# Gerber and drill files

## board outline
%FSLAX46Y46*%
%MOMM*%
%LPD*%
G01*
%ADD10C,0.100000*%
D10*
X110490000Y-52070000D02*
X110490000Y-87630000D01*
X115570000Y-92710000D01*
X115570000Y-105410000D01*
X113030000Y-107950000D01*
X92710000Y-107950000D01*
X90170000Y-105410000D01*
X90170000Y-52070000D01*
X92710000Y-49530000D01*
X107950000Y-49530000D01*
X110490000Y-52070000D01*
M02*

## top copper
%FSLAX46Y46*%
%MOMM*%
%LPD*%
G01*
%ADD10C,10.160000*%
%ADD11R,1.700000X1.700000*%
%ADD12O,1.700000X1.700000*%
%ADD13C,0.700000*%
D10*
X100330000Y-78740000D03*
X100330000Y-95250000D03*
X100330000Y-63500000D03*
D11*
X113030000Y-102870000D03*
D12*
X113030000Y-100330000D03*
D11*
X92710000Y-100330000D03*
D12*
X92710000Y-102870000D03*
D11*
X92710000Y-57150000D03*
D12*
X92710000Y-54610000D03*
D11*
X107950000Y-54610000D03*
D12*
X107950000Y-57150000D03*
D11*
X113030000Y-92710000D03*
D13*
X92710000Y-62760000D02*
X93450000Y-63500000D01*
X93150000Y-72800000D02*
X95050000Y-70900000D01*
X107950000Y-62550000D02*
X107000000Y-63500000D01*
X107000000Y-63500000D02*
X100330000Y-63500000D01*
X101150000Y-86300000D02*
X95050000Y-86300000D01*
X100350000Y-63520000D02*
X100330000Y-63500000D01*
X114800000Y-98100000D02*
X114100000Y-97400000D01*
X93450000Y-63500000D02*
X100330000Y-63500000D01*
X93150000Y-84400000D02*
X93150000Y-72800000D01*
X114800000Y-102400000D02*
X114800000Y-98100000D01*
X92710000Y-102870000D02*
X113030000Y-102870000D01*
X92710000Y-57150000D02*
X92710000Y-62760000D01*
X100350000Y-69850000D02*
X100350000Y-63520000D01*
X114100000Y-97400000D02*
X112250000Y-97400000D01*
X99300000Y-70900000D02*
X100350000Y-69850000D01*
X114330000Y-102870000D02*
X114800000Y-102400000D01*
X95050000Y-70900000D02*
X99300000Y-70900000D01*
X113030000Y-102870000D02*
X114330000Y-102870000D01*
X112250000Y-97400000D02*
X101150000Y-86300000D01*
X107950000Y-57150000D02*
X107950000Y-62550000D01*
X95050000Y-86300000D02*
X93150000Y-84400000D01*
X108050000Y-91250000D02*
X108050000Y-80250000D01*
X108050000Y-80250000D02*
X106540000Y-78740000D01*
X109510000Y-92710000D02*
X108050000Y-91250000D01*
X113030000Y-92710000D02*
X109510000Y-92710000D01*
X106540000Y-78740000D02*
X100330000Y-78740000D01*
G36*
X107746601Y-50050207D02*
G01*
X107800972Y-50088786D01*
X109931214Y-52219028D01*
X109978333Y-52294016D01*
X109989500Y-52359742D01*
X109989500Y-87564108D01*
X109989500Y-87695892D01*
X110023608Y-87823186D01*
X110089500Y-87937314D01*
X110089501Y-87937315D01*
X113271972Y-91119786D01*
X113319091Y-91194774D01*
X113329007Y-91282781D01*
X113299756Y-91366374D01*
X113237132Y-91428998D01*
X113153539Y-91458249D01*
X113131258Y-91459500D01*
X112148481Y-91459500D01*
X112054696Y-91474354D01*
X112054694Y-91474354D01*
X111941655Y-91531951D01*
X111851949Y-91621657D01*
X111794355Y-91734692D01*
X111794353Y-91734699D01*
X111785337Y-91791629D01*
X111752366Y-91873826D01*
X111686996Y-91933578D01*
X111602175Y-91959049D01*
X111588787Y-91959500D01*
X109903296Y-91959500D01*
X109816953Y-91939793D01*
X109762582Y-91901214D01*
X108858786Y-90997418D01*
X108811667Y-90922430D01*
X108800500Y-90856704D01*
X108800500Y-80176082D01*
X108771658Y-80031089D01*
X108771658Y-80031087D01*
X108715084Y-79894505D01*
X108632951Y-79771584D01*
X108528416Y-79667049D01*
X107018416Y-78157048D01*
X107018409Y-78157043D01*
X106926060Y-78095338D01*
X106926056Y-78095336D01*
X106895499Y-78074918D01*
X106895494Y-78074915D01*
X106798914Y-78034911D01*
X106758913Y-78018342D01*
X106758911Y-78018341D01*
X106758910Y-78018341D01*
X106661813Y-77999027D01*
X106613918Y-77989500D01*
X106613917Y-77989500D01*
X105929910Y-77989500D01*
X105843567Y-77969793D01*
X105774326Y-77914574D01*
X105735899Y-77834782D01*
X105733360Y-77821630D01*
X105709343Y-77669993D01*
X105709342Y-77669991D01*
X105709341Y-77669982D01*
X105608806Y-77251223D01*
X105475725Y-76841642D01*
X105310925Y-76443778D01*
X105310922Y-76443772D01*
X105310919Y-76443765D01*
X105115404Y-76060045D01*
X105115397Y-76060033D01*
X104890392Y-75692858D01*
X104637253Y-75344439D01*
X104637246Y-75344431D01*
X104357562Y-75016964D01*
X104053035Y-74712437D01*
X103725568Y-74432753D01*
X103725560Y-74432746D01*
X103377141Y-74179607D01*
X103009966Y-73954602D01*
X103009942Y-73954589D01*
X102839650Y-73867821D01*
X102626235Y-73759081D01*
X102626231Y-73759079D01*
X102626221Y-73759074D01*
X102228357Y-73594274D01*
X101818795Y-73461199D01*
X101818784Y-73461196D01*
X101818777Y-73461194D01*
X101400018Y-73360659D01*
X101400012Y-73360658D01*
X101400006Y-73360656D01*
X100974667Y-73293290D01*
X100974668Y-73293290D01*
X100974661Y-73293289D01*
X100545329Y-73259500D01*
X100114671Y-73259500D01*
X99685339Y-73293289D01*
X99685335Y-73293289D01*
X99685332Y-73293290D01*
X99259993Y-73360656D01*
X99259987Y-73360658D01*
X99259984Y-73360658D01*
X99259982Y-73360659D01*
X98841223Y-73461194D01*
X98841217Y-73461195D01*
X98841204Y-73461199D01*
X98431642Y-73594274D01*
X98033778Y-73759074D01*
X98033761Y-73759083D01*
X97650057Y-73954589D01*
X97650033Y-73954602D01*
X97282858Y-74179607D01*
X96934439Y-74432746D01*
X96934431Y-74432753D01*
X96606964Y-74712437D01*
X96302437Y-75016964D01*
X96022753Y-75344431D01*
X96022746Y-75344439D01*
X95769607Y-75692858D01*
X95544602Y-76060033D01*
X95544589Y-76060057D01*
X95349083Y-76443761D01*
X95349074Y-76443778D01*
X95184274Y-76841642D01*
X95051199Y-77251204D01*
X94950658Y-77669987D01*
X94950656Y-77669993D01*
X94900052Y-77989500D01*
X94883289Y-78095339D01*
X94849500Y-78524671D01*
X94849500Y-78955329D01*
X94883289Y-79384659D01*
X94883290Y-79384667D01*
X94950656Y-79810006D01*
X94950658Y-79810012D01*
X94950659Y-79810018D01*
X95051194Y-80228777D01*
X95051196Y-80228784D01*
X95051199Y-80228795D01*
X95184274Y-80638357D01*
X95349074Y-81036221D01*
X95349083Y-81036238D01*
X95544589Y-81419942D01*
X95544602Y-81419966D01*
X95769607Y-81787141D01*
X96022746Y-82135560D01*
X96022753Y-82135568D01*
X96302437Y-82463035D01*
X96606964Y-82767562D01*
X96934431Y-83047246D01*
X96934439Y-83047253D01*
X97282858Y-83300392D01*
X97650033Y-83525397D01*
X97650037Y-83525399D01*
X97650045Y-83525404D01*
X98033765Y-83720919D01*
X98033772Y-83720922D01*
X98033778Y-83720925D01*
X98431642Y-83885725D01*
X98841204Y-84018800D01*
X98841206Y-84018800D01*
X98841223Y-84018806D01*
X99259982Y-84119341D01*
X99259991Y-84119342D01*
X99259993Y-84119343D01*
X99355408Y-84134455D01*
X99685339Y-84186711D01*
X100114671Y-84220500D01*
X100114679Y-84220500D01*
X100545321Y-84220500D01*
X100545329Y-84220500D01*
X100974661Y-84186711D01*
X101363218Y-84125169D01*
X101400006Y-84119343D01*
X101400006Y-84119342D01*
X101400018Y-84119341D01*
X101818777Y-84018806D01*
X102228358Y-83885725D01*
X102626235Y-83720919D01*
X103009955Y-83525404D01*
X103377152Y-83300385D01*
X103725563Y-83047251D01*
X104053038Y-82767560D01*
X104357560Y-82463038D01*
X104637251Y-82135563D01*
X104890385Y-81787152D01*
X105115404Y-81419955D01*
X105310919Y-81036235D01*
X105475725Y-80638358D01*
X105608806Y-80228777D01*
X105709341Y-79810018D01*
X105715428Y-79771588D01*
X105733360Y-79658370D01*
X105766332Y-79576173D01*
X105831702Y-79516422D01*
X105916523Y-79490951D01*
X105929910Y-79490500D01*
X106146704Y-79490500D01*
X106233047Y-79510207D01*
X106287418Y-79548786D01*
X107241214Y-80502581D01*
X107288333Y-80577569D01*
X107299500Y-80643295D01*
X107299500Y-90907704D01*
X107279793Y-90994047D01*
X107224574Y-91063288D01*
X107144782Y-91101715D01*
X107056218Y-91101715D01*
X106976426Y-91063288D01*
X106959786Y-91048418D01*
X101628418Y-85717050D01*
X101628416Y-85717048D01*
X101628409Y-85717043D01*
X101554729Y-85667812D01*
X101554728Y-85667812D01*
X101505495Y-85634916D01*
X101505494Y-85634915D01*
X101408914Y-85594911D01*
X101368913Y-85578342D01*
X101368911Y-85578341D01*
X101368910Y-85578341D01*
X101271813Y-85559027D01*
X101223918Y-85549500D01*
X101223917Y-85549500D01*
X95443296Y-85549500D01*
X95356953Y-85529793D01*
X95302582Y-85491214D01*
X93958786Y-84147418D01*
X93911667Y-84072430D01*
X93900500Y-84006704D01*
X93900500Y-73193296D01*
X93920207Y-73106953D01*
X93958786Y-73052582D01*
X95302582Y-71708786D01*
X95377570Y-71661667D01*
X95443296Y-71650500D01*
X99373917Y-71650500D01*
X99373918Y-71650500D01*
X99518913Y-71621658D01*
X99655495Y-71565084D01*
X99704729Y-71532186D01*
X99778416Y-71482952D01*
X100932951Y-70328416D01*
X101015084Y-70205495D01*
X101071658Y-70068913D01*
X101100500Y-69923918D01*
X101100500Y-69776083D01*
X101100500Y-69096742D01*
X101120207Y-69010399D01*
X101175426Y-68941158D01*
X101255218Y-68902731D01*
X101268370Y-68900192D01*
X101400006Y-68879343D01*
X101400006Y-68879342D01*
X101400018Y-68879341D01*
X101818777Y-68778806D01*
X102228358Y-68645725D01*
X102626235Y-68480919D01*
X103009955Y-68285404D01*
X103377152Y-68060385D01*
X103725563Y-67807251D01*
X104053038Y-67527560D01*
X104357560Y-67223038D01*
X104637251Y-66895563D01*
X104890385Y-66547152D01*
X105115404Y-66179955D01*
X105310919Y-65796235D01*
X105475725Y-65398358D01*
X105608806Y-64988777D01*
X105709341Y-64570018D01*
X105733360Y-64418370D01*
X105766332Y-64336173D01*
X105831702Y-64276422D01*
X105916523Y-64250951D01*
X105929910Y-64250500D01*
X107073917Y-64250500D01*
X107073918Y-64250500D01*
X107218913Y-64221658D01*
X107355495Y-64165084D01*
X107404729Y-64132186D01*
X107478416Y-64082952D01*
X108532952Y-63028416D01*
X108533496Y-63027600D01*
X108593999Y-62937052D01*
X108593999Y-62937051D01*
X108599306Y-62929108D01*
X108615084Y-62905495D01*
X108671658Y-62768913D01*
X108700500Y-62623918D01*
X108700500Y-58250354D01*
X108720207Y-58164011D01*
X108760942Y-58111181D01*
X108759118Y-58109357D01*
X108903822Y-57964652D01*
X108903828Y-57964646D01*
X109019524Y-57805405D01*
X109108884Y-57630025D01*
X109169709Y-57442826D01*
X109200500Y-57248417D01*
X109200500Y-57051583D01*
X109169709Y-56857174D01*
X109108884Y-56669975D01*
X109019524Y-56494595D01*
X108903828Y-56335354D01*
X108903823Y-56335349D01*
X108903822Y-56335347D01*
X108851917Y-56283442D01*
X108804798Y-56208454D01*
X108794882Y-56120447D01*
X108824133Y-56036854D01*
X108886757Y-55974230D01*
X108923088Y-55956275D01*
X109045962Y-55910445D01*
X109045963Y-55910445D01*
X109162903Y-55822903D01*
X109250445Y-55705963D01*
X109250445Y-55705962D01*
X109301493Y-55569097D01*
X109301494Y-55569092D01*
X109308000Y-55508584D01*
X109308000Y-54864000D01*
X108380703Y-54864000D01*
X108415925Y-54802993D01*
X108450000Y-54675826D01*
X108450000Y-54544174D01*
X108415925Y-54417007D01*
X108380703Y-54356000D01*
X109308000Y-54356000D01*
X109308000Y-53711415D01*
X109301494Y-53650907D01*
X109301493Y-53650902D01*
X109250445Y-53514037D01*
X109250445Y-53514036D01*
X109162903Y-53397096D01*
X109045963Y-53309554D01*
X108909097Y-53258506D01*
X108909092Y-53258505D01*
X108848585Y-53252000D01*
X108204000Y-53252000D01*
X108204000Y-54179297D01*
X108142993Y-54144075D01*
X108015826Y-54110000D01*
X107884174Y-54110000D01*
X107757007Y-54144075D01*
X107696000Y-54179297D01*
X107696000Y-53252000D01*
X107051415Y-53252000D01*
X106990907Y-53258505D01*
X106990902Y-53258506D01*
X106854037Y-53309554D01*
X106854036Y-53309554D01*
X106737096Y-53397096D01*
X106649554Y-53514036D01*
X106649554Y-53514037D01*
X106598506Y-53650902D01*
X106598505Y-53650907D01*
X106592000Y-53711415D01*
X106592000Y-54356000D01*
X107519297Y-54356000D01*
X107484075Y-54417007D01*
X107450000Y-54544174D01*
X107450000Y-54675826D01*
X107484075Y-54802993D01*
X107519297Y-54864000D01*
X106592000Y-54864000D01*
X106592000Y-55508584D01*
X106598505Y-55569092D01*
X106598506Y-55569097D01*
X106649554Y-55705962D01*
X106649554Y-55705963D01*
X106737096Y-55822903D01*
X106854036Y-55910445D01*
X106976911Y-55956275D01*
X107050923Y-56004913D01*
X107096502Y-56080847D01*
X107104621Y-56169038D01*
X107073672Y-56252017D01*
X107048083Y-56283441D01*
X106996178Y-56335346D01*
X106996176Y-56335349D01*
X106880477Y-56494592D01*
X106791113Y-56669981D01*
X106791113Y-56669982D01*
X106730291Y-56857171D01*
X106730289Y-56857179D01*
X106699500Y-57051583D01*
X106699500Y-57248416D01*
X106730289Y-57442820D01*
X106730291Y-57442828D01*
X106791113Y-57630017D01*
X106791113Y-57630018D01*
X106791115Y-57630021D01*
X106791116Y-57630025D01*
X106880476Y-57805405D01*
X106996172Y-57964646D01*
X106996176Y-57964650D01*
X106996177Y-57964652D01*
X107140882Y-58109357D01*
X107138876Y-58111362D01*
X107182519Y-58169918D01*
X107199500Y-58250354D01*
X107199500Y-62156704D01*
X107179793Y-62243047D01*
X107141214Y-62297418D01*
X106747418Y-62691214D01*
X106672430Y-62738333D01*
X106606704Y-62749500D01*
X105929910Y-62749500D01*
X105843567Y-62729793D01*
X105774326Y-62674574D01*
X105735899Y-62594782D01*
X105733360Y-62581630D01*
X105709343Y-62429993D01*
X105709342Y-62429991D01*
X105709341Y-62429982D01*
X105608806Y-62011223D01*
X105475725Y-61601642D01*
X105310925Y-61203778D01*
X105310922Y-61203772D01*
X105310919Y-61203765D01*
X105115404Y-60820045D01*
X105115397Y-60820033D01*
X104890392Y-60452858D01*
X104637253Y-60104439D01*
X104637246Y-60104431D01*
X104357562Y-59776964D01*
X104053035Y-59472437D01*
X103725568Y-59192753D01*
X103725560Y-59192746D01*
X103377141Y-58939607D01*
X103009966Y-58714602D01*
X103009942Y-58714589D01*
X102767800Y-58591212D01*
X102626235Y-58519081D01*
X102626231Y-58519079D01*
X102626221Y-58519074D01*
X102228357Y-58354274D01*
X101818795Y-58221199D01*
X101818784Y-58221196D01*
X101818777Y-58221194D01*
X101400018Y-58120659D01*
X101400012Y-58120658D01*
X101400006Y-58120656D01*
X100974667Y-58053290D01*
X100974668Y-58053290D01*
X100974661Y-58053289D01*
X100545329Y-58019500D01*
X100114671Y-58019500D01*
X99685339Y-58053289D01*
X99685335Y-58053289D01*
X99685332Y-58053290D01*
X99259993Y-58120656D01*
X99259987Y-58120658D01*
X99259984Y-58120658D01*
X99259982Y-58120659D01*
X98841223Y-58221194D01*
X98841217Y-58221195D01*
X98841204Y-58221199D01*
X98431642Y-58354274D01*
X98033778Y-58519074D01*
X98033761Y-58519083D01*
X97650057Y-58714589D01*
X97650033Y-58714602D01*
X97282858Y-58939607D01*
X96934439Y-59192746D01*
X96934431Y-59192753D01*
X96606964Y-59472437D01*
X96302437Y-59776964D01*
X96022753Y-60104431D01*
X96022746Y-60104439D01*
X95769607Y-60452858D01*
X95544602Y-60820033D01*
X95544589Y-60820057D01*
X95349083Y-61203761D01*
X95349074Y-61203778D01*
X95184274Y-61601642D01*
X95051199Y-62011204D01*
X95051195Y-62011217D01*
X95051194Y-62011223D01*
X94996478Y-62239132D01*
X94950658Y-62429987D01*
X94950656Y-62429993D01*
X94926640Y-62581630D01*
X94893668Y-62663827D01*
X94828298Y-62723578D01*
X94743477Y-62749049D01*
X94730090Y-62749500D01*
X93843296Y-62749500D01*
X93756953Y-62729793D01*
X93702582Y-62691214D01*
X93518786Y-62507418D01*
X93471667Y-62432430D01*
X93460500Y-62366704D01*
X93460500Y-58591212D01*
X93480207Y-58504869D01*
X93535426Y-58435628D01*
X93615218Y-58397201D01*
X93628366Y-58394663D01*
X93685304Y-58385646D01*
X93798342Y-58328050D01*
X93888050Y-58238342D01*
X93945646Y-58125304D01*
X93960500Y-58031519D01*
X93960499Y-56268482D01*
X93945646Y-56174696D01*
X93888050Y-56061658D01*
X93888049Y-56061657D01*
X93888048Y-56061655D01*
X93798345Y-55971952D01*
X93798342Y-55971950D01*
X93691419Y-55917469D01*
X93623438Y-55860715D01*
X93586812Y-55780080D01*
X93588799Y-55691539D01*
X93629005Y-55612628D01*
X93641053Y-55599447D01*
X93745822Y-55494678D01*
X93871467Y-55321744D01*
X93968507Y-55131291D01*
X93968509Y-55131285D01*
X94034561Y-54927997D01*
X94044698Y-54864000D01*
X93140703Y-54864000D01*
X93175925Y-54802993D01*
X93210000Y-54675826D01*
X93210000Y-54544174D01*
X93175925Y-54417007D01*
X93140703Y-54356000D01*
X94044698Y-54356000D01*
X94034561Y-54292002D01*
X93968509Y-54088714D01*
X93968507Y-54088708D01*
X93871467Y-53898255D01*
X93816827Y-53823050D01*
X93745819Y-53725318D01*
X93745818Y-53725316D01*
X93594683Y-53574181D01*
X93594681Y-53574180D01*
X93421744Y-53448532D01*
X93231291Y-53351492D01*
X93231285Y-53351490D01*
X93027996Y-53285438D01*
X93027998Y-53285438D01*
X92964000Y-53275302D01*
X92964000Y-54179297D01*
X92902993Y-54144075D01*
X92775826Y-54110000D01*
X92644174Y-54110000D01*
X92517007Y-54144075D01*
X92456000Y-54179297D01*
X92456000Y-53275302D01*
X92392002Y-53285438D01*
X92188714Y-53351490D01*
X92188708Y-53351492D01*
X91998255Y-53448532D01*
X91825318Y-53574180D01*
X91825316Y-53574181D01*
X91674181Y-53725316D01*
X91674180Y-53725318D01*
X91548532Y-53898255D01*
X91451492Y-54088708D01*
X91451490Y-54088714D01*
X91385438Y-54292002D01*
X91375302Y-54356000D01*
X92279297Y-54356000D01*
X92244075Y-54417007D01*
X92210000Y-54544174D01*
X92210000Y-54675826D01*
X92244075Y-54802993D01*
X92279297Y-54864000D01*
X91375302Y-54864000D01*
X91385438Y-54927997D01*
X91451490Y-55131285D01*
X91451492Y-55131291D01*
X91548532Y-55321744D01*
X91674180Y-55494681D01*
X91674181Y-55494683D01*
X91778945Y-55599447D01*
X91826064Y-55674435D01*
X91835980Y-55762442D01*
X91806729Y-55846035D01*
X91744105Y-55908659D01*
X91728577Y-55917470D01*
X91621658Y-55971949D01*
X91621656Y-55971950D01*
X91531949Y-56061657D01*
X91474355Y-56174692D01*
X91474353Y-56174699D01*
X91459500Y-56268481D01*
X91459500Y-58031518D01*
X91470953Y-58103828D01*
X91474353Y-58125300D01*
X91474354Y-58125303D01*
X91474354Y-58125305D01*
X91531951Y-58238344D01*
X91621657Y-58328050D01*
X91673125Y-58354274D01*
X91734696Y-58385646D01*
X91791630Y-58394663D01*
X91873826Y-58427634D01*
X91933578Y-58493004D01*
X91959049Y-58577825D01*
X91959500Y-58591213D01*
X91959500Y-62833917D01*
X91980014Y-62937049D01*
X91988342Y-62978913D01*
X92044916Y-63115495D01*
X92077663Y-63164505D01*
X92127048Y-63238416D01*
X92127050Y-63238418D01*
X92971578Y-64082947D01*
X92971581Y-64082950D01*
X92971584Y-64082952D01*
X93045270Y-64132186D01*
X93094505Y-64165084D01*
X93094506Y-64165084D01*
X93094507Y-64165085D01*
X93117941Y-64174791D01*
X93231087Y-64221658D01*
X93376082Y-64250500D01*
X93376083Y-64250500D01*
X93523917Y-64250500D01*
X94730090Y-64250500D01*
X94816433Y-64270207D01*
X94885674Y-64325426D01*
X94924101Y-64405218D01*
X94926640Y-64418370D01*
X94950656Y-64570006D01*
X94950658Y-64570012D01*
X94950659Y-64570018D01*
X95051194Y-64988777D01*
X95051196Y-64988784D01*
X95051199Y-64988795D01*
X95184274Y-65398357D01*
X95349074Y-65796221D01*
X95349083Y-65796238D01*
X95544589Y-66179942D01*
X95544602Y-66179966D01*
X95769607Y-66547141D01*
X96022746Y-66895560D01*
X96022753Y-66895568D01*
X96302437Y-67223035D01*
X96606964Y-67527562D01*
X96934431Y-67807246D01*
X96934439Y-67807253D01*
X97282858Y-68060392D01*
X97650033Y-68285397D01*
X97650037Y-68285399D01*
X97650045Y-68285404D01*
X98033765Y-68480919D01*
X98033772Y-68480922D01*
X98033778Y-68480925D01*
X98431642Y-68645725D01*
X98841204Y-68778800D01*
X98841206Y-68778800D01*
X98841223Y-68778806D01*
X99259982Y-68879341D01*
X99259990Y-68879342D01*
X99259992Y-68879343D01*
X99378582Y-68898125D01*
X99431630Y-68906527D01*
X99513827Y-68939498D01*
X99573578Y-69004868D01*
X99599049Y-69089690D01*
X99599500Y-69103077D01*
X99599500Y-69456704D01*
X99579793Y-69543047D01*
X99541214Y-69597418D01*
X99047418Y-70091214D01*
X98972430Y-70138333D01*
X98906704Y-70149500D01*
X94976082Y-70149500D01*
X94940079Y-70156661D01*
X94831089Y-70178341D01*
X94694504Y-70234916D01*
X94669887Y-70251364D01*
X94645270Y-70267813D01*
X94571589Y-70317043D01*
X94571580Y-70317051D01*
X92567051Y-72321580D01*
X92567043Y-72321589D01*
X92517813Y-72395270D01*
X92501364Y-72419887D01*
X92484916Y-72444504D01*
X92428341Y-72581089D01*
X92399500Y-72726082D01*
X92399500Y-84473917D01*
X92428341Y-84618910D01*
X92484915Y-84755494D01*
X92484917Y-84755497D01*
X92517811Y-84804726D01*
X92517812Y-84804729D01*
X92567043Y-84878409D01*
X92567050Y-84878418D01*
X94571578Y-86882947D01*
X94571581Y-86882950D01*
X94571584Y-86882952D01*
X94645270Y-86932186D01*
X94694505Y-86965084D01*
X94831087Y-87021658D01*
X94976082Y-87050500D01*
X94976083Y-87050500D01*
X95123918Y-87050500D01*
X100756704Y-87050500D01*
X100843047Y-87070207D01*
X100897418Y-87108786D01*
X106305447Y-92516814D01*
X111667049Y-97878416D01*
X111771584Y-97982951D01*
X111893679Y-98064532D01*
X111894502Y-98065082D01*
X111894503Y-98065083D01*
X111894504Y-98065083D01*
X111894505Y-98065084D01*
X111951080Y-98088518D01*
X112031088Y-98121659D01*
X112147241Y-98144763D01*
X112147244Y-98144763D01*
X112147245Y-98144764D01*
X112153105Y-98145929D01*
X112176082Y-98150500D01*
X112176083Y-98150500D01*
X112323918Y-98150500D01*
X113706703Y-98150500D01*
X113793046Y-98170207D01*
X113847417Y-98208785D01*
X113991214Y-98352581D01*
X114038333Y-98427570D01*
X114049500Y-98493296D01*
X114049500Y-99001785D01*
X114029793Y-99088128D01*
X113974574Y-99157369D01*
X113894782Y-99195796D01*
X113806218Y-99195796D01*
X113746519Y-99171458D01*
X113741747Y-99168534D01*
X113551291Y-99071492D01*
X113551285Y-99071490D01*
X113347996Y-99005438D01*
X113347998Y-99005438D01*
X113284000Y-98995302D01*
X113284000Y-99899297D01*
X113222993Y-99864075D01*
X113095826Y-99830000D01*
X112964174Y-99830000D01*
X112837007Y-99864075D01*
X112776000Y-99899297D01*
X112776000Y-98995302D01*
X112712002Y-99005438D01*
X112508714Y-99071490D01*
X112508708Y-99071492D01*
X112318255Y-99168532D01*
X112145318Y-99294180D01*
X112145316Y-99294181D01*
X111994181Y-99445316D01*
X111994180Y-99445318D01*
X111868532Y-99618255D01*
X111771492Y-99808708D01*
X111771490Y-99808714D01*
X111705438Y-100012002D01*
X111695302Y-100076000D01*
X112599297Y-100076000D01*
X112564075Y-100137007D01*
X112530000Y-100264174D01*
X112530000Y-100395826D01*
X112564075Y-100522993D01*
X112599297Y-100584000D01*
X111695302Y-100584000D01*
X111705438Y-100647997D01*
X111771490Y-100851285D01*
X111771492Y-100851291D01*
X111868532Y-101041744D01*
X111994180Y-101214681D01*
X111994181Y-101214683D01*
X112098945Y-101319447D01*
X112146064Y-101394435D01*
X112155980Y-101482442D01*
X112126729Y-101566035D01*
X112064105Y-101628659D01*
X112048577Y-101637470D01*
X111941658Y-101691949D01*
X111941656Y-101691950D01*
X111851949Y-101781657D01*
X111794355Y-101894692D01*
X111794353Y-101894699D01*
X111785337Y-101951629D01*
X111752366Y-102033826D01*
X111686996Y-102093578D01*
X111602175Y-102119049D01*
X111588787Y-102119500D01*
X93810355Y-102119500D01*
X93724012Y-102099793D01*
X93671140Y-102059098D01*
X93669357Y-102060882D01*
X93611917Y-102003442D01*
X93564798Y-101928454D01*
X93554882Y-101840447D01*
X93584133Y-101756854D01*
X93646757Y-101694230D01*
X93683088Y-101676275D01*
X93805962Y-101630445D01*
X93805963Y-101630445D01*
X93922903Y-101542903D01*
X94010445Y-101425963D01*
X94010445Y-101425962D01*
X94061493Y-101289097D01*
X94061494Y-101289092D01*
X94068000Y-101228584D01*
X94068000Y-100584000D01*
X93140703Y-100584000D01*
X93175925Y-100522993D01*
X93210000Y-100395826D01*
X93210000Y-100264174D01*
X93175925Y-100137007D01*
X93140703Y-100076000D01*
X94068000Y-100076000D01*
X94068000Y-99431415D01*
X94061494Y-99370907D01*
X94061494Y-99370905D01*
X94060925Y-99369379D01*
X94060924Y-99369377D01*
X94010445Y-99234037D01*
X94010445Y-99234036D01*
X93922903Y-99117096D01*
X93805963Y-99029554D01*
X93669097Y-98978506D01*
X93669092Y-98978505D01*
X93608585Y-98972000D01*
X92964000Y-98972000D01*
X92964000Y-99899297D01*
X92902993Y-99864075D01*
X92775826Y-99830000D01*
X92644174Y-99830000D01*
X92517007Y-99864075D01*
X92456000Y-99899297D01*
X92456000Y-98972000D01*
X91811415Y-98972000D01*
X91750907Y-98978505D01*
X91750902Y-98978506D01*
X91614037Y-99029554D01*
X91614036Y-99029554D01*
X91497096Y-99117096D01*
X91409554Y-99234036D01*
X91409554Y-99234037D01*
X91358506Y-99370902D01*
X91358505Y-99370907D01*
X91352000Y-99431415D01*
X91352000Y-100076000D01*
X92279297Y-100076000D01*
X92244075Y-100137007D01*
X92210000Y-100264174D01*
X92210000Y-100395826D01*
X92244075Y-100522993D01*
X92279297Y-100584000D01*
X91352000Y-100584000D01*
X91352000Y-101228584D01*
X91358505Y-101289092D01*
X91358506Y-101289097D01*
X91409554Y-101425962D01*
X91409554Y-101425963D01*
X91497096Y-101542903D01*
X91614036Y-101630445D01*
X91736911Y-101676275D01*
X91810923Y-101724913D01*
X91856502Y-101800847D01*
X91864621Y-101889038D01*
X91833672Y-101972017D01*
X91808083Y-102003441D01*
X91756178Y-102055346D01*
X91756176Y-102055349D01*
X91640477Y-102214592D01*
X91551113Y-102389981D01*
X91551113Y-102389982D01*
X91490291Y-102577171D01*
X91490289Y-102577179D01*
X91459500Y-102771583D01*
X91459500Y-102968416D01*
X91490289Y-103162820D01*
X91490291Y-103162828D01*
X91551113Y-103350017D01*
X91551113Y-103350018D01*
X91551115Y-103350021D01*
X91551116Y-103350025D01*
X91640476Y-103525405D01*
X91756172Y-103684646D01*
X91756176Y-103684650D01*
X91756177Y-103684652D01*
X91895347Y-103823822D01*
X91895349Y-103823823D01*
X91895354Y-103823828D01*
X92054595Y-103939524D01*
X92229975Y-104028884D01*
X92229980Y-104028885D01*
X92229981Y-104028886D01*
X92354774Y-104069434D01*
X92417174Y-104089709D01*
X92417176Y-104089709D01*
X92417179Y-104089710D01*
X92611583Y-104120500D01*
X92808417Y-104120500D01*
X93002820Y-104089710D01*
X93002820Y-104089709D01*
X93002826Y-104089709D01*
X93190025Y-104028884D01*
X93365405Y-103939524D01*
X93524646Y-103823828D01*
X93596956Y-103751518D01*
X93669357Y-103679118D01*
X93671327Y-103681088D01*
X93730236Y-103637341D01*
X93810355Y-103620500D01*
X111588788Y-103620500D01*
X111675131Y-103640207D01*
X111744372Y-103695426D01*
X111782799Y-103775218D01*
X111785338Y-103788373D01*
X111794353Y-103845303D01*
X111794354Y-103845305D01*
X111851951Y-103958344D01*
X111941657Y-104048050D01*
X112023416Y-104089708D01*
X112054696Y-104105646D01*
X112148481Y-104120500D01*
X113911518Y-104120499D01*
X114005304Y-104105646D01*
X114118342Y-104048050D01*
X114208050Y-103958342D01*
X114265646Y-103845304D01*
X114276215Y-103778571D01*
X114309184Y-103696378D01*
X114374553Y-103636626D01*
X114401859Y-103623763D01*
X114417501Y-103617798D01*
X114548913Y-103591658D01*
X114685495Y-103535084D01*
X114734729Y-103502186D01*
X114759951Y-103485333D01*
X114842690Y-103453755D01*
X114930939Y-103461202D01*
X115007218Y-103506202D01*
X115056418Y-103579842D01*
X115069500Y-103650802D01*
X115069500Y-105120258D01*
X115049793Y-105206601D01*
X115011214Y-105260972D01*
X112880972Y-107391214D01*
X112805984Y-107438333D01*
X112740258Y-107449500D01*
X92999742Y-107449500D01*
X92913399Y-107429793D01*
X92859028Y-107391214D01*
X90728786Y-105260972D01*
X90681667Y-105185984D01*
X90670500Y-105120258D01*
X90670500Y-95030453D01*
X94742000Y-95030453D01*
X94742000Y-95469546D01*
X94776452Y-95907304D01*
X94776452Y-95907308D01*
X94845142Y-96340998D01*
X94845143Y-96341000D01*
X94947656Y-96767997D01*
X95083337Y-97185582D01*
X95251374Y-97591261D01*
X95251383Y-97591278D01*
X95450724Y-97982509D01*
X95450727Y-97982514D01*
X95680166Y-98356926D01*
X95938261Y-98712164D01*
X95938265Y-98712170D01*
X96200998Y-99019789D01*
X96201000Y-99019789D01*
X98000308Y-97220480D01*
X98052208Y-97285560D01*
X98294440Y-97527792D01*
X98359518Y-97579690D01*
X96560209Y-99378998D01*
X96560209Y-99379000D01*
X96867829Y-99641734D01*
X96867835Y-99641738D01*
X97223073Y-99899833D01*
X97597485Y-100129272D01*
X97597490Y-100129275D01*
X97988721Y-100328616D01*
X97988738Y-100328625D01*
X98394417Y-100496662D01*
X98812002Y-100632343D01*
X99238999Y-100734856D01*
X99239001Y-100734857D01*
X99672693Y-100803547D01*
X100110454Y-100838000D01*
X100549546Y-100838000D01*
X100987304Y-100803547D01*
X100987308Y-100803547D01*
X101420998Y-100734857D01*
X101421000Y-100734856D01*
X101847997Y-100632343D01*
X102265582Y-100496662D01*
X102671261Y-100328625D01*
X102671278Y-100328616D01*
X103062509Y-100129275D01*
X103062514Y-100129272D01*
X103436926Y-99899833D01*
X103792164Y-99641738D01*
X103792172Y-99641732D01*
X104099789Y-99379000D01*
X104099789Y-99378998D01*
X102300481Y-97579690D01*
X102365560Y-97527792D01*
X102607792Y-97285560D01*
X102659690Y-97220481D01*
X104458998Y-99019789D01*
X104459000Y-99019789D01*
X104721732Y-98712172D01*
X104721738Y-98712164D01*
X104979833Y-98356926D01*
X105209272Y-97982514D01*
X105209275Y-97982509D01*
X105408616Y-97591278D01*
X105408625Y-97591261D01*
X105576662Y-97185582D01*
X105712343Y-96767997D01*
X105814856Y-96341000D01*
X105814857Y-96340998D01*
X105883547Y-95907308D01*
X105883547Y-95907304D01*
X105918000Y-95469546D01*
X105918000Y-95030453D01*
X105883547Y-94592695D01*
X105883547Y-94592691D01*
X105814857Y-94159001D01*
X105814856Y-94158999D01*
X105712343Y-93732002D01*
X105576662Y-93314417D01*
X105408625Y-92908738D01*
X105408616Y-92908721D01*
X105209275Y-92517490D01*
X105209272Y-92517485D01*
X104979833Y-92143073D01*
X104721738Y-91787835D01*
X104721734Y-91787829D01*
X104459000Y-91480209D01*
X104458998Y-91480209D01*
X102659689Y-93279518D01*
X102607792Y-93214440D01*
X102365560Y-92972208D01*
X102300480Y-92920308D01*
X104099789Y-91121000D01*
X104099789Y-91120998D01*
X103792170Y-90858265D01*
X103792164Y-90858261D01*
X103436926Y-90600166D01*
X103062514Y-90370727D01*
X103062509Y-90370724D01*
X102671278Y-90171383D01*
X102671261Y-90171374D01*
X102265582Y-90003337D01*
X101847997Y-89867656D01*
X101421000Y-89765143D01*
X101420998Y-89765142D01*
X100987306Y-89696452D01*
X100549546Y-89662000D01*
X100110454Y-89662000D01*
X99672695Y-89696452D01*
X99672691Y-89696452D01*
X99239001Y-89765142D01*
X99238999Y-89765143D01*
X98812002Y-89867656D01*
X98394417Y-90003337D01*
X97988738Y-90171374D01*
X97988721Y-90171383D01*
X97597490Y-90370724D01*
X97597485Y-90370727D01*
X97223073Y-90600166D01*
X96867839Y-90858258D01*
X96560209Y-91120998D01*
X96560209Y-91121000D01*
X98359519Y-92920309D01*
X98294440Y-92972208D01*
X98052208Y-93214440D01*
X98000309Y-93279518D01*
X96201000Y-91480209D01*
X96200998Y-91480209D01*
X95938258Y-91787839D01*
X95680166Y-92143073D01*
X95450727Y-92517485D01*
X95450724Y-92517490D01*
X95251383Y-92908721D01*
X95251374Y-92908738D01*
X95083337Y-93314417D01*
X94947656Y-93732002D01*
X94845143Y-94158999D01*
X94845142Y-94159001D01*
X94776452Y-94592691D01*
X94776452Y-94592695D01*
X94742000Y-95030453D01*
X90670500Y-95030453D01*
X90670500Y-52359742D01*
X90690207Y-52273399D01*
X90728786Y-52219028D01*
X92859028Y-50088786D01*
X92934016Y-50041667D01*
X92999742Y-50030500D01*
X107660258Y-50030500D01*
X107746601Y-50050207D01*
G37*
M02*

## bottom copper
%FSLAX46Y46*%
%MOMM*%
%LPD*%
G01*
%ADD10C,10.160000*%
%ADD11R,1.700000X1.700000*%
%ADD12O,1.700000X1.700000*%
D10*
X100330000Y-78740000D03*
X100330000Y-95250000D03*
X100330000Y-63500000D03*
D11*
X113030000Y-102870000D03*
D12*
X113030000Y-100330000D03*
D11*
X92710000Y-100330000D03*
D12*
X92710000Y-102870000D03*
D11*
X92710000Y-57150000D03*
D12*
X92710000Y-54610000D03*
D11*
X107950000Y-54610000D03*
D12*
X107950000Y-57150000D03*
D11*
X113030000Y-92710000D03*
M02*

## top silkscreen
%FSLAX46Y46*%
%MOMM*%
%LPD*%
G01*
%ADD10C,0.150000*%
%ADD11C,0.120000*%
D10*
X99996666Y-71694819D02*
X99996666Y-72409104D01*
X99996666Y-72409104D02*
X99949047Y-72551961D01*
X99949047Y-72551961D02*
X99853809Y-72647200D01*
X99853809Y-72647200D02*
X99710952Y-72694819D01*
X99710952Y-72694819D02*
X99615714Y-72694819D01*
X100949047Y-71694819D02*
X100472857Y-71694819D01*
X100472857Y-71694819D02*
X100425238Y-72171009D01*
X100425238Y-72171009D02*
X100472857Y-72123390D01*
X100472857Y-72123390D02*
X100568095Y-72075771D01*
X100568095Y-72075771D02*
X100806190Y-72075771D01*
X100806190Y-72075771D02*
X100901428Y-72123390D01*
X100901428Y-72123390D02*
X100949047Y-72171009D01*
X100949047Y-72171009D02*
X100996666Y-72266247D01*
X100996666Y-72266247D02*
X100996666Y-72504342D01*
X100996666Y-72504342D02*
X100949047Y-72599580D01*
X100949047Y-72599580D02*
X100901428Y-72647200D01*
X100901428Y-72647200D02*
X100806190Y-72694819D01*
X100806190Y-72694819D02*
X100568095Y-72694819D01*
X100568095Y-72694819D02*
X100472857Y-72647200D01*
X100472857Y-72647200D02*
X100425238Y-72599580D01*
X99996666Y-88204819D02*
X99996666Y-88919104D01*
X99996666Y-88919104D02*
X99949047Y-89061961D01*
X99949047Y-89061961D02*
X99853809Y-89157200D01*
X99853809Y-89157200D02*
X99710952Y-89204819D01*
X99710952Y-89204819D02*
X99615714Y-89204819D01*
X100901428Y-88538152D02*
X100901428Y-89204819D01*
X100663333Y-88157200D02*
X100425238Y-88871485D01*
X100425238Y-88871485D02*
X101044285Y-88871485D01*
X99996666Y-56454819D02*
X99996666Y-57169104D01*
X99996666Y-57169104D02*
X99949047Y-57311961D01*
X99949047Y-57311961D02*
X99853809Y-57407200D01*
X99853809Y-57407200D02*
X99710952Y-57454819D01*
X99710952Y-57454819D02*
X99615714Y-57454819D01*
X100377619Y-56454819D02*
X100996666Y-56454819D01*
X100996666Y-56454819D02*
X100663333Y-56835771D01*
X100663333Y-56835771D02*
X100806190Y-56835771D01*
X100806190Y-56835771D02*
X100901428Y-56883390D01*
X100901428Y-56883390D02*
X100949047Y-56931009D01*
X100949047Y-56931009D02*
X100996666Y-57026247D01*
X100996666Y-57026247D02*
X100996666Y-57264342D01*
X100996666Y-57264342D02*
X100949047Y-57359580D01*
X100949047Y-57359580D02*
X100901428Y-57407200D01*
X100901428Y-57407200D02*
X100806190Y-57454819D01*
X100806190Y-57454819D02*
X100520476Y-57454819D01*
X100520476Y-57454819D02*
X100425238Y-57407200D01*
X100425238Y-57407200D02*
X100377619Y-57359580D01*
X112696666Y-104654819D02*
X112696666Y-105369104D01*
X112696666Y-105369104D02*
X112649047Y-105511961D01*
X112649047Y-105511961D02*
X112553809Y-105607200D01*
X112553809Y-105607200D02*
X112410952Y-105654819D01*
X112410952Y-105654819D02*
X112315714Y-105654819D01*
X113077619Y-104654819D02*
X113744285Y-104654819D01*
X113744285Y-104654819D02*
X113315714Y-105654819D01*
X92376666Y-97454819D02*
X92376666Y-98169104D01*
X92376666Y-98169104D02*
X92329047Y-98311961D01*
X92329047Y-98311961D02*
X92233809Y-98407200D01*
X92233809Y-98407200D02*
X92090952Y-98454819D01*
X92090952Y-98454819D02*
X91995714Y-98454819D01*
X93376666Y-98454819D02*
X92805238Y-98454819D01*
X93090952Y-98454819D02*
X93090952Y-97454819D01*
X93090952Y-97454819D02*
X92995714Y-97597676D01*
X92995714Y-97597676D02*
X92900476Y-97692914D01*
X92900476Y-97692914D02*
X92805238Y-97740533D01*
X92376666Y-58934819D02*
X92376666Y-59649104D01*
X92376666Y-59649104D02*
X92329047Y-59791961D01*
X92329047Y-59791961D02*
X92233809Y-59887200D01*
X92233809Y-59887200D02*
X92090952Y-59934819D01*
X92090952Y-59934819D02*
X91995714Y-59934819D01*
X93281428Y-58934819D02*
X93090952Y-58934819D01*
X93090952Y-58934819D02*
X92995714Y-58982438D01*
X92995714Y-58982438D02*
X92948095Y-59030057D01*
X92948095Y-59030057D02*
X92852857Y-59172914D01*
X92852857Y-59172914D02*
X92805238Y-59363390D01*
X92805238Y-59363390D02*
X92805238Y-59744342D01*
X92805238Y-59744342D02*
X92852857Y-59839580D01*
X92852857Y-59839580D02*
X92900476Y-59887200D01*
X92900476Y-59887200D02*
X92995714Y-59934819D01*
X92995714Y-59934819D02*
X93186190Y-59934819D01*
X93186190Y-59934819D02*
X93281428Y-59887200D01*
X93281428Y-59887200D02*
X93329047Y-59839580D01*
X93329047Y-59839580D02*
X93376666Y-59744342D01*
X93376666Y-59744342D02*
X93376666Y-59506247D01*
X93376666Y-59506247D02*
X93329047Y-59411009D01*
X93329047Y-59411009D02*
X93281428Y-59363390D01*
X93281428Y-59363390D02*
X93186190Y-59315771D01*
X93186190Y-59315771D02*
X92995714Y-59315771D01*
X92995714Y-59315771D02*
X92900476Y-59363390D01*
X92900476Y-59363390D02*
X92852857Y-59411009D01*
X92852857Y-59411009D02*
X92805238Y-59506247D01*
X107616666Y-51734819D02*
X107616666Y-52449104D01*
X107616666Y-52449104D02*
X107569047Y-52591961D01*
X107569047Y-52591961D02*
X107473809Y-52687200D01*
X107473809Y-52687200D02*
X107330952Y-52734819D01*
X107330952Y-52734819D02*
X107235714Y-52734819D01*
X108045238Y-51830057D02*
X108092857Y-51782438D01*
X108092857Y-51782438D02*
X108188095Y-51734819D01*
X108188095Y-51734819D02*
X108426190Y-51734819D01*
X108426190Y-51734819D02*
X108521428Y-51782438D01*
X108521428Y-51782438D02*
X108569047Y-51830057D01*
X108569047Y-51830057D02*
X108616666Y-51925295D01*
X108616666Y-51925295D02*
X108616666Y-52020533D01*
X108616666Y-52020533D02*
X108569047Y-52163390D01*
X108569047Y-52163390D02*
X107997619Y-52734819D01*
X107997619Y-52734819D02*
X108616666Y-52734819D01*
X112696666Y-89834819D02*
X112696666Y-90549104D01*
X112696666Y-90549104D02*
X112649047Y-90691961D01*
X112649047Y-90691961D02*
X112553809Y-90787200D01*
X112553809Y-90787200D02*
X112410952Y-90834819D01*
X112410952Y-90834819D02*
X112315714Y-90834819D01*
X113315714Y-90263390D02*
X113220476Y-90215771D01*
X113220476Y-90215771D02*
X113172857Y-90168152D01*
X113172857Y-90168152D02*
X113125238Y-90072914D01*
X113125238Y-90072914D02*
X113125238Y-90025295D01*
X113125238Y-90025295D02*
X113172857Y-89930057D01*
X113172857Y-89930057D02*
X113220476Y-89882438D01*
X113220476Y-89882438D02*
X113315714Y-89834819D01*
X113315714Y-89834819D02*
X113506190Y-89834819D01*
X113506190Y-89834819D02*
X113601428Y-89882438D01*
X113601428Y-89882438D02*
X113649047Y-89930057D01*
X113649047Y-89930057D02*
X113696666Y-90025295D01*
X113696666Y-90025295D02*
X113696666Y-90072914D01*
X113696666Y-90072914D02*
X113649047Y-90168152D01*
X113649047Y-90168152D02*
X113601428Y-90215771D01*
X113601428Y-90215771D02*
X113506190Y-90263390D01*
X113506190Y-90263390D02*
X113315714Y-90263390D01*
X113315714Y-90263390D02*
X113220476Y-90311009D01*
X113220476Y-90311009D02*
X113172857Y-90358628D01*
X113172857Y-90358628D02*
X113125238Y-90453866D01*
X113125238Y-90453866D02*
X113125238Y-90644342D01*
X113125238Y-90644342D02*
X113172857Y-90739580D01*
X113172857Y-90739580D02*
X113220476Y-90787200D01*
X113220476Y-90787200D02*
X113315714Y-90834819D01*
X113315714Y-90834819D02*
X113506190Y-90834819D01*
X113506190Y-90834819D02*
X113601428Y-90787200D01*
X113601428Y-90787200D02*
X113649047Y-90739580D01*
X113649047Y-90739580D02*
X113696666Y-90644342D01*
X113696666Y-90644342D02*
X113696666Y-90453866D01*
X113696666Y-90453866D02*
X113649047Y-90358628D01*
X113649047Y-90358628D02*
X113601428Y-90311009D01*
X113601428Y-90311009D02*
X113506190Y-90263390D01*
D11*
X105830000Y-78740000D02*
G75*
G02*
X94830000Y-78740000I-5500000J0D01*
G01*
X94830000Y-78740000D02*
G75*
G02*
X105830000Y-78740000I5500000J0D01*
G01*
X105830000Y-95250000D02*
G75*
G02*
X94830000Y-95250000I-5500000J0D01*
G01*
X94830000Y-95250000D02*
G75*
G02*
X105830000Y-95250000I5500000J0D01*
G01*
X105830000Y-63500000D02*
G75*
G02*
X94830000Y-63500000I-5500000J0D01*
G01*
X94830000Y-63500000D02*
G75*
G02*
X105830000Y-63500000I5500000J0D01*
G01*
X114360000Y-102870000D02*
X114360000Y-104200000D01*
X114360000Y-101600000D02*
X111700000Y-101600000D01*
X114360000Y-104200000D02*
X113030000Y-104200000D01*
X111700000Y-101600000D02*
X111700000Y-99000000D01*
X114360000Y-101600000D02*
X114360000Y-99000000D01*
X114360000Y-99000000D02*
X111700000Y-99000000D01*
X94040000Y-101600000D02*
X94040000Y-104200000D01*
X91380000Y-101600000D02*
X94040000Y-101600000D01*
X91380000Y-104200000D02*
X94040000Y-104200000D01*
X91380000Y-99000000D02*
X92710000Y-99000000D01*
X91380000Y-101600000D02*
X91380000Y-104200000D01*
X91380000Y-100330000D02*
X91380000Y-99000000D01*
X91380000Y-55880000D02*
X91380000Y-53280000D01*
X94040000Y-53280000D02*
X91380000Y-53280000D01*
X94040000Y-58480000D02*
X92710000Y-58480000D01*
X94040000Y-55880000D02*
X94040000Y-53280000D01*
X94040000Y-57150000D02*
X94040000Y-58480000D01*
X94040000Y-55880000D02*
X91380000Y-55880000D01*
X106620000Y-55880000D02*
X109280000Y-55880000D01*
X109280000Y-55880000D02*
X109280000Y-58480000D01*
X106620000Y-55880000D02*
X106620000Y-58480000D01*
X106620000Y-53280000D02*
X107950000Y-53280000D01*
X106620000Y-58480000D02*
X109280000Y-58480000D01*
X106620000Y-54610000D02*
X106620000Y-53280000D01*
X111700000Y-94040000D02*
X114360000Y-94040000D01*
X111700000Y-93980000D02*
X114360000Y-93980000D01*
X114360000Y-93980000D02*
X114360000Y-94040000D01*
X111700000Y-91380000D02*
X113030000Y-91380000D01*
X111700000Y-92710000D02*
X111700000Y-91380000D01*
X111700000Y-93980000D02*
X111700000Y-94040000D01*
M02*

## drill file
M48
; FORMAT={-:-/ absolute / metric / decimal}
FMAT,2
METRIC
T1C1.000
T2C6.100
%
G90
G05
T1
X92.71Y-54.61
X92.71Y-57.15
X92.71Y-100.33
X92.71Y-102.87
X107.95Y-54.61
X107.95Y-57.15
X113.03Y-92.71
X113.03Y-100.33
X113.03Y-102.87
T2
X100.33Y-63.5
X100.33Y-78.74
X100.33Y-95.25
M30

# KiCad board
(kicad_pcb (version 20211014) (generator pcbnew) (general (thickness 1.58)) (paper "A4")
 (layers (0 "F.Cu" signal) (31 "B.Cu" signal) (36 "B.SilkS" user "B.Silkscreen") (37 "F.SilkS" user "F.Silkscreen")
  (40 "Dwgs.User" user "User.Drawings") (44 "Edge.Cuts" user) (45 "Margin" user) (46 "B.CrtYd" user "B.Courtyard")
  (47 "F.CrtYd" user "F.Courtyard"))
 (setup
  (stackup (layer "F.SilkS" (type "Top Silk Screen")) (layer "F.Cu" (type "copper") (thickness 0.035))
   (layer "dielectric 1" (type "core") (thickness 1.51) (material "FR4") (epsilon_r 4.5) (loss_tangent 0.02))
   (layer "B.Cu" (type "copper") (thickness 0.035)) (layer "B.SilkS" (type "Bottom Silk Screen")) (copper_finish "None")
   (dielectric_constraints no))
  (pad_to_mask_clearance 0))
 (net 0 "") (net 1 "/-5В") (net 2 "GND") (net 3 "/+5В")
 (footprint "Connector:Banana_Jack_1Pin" (layer "F.Cu") (at 100.33 78.74)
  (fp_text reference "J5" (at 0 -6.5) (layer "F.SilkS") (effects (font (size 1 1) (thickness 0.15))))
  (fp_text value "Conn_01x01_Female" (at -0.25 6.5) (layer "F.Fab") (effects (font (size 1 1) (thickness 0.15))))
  (fp_circle (center 0 0) (end 5.5 0) (layer "F.SilkS") (width 0.12) (fill none))
  (pad "1" thru_hole circle (at 0 0) (size 10.16 10.16) (drill 6.1) (layers *.Cu *.Mask) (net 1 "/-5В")))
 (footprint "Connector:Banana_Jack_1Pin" (layer "F.Cu") (at 100.33 95.25)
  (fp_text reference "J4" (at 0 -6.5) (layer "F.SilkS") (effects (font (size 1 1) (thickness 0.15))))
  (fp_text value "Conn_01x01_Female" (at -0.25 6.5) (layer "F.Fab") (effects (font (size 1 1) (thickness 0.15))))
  (fp_circle (center 0 0) (end 5.5 0) (layer "F.SilkS") (width 0.12) (fill none))
  (pad "1" thru_hole circle (at 0 0) (size 10.16 10.16) (drill 6.1) (layers *.Cu *.Mask) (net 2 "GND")))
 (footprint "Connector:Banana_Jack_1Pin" (layer "F.Cu") (at 100.33 63.5)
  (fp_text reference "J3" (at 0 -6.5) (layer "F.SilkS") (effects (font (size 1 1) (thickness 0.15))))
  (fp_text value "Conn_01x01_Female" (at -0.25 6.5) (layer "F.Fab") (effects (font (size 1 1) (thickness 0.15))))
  (fp_circle (center 0 0) (end 5.5 0) (layer "F.SilkS") (width 0.12) (fill none))
  (pad "1" thru_hole circle (at 0 0) (size 10.16 10.16) (drill 6.1) (layers *.Cu *.Mask) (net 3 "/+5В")))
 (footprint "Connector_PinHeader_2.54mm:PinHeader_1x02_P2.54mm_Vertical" (layer "F.Cu") (at 113.03 102.87 180)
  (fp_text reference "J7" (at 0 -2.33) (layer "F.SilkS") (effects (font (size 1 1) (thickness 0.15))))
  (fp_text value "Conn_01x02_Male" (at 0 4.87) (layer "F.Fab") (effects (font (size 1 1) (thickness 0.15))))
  (fp_line (start -1.33 0) (end -1.33 -1.33) (layer "F.SilkS") (width 0.12))
  (fp_line (start -1.33 1.27) (end 1.33 1.27) (layer "F.SilkS") (width 0.12))
  (fp_line (start -1.33 -1.33) (end 0 -1.33) (layer "F.SilkS") (width 0.12))
  (fp_line (start 1.33 1.27) (end 1.33 3.87) (layer "F.SilkS") (width 0.12))
  (fp_line (start -1.33 1.27) (end -1.33 3.87) (layer "F.SilkS") (width 0.12))
  (fp_line (start -1.33 3.87) (end 1.33 3.87) (layer "F.SilkS") (width 0.12))
  (pad "1" thru_hole rect (at 0 0 180) (size 1.7 1.7) (drill 1) (layers *.Cu *.Mask) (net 3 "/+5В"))
  (pad "2" thru_hole oval (at 0 2.54 180) (size 1.7 1.7) (drill 1) (layers *.Cu *.Mask) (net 2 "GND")))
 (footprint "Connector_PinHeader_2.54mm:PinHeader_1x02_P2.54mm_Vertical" (layer "F.Cu") (at 92.71 100.33)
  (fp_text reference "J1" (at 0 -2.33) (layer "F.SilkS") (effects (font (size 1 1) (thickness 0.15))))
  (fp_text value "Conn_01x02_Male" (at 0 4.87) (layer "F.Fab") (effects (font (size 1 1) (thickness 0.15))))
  (fp_line (start 1.33 1.27) (end 1.33 3.87) (layer "F.SilkS") (width 0.12))
  (fp_line (start -1.33 1.27) (end 1.33 1.27) (layer "F.SilkS") (width 0.12))
  (fp_line (start -1.33 3.87) (end 1.33 3.87) (layer "F.SilkS") (width 0.12))
  (fp_line (start -1.33 -1.33) (end 0 -1.33) (layer "F.SilkS") (width 0.12))
  (fp_line (start -1.33 1.27) (end -1.33 3.87) (layer "F.SilkS") (width 0.12))
  (fp_line (start -1.33 0) (end -1.33 -1.33) (layer "F.SilkS") (width 0.12))
  (pad "1" thru_hole rect (at 0 0) (size 1.7 1.7) (drill 1) (layers *.Cu *.Mask) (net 2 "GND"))
  (pad "2" thru_hole oval (at 0 2.54) (size 1.7 1.7) (drill 1) (layers *.Cu *.Mask) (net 3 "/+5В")))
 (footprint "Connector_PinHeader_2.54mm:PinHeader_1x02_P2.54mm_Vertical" (layer "F.Cu") (at 92.71 57.15 180)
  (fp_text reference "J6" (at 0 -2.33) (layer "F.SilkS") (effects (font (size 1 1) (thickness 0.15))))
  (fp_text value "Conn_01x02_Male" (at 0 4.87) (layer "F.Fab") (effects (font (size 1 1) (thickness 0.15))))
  (fp_line (start 1.33 1.27) (end 1.33 3.87) (layer "F.SilkS") (width 0.12))
  (fp_line (start -1.33 3.87) (end 1.33 3.87) (layer "F.SilkS") (width 0.12))
  (fp_line (start -1.33 -1.33) (end 0 -1.33) (layer "F.SilkS") (width 0.12))
  (fp_line (start -1.33 1.27) (end -1.33 3.87) (layer "F.SilkS") (width 0.12))
  (fp_line (start -1.33 0) (end -1.33 -1.33) (layer "F.SilkS") (width 0.12))
  (fp_line (start -1.33 1.27) (end 1.33 1.27) (layer "F.SilkS") (width 0.12))
  (pad "1" thru_hole rect (at 0 0 180) (size 1.7 1.7) (drill 1) (layers *.Cu *.Mask) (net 3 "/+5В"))
  (pad "2" thru_hole oval (at 0 2.54 180) (size 1.7 1.7) (drill 1) (layers *.Cu *.Mask) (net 2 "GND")))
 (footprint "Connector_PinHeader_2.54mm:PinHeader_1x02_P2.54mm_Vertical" (layer "F.Cu") (at 107.95 54.61)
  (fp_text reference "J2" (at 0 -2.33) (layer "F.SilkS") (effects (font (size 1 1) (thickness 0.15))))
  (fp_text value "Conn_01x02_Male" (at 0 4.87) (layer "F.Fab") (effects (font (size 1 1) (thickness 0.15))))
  (fp_line (start -1.33 1.27) (end 1.33 1.27) (layer "F.SilkS") (width 0.12))
  (fp_line (start 1.33 1.27) (end 1.33 3.87) (layer "F.SilkS") (width 0.12))
  (fp_line (start -1.33 1.27) (end -1.33 3.87) (layer "F.SilkS") (width 0.12))
  (fp_line (start -1.33 -1.33) (end 0 -1.33) (layer "F.SilkS") (width 0.12))
  (fp_line (start -1.33 3.87) (end 1.33 3.87) (layer "F.SilkS") (width 0.12))
  (fp_line (start -1.33 0) (end -1.33 -1.33) (layer "F.SilkS") (width 0.12))
  (pad "1" thru_hole rect (at 0 0) (size 1.7 1.7) (drill 1) (layers *.Cu *.Mask) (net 2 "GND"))
  (pad "2" thru_hole oval (at 0 2.54) (size 1.7 1.7) (drill 1) (layers *.Cu *.Mask) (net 3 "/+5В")))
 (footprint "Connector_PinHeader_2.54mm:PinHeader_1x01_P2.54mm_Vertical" (layer "F.Cu") (at 113.03 92.71)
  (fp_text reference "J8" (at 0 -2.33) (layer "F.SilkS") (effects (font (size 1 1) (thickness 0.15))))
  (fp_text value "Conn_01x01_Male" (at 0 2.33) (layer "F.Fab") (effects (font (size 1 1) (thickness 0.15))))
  (fp_line (start -1.33 1.33) (end 1.33 1.33) (layer "F.SilkS") (width 0.12))
  (fp_line (start -1.33 1.27) (end 1.33 1.27) (layer "F.SilkS") (width 0.12))
  (fp_line (start 1.33 1.27) (end 1.33 1.33) (layer "F.SilkS") (width 0.12))
  (fp_line (start -1.33 -1.33) (end 0 -1.33) (layer "F.SilkS") (width 0.12))
  (fp_line (start -1.33 0) (end -1.33 -1.33) (layer "F.SilkS") (width 0.12))
  (fp_line (start -1.33 1.27) (end -1.33 1.33) (layer "F.SilkS") (width 0.12))
  (pad "1" thru_hole rect (at 0 0) (size 1.7 1.7) (drill 1) (layers *.Cu *.Mask) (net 1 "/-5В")))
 (gr_poly
  (pts (xy 110.49 52.07) (xy 110.49 87.63) (xy 115.57 92.71) (xy 115.57 105.41) (xy 113.03 107.95) (xy 92.71 107.95) (xy 90.17 105.41)
   (xy 90.17 52.07) (xy 92.71 49.53) (xy 107.95 49.53))
  (layer "Edge.Cuts") (width 0.1) (fill none))
 (segment (start 92.71 62.76) (end 93.45 63.5) (width 0.7) (layer "F.Cu") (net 3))
 (segment (start 93.15 72.8) (end 95.05 70.9) (width 0.7) (layer "F.Cu") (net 3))
 (segment (start 107.95 62.55) (end 107 63.5) (width 0.7) (layer "F.Cu") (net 3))
 (segment (start 107 63.5) (end 100.33 63.5) (width 0.7) (layer "F.Cu") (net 3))
 (segment (start 101.15 86.3) (end 95.05 86.3) (width 0.7) (layer "F.Cu") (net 3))
 (segment (start 100.35 63.52) (end 100.33 63.5) (width 0.7) (layer "F.Cu") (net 3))
 (segment (start 114.8 98.1) (end 114.1 97.4) (width 0.7) (layer "F.Cu") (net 3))
 (segment (start 93.45 63.5) (end 100.33 63.5) (width 0.7) (layer "F.Cu") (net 3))
 (segment (start 93.15 84.4) (end 93.15 72.8) (width 0.7) (layer "F.Cu") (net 3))
 (segment (start 114.8 102.4) (end 114.8 98.1) (width 0.7) (layer "F.Cu") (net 3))
 (segment (start 92.71 102.87) (end 113.03 102.87) (width 0.7) (layer "F.Cu") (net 3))
 (segment (start 92.71 57.15) (end 92.71 62.76) (width 0.7) (layer "F.Cu") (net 3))
 (segment (start 100.35 69.85) (end 100.35 63.52) (width 0.7) (layer "F.Cu") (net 3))
 (segment (start 114.1 97.4) (end 112.25 97.4) (width 0.7) (layer "F.Cu") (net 3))
 (segment (start 99.3 70.9) (end 100.35 69.85) (width 0.7) (layer "F.Cu") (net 3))
 (segment (start 114.33 102.87) (end 114.8 102.4) (width 0.7) (layer "F.Cu") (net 3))
 (segment (start 95.05 70.9) (end 99.3 70.9) (width 0.7) (layer "F.Cu") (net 3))
 (segment (start 113.03 102.87) (end 114.33 102.87) (width 0.7) (layer "F.Cu") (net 3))
 (segment (start 112.25 97.4) (end 101.15 86.3) (width 0.7) (layer "F.Cu") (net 3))
 (segment (start 107.95 57.15) (end 107.95 62.55) (width 0.7) (layer "F.Cu") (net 3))
 (segment (start 95.05 86.3) (end 93.15 84.4) (width 0.7) (layer "F.Cu") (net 3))
 (segment (start 108.05 91.25) (end 108.05 80.25) (width 0.7) (layer "F.Cu") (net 1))
 (segment (start 108.05 80.25) (end 106.54 78.74) (width 0.7) (layer "F.Cu") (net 1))
 (segment (start 109.51 92.71) (end 108.05 91.25) (width 0.7) (layer "F.Cu") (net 1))
 (segment (start 113.03 92.71) (end 109.51 92.71) (width 0.7) (layer "F.Cu") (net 1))
 (segment (start 106.54 78.74) (end 100.33 78.74) (width 0.7) (layer "F.Cu") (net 1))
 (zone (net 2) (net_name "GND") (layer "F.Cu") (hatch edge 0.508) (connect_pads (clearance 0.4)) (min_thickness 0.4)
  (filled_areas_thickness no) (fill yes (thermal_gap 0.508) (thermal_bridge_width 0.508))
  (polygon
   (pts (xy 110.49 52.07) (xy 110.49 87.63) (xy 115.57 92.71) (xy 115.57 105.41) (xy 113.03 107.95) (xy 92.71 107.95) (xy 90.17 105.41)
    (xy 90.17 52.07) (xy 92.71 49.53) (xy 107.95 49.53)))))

